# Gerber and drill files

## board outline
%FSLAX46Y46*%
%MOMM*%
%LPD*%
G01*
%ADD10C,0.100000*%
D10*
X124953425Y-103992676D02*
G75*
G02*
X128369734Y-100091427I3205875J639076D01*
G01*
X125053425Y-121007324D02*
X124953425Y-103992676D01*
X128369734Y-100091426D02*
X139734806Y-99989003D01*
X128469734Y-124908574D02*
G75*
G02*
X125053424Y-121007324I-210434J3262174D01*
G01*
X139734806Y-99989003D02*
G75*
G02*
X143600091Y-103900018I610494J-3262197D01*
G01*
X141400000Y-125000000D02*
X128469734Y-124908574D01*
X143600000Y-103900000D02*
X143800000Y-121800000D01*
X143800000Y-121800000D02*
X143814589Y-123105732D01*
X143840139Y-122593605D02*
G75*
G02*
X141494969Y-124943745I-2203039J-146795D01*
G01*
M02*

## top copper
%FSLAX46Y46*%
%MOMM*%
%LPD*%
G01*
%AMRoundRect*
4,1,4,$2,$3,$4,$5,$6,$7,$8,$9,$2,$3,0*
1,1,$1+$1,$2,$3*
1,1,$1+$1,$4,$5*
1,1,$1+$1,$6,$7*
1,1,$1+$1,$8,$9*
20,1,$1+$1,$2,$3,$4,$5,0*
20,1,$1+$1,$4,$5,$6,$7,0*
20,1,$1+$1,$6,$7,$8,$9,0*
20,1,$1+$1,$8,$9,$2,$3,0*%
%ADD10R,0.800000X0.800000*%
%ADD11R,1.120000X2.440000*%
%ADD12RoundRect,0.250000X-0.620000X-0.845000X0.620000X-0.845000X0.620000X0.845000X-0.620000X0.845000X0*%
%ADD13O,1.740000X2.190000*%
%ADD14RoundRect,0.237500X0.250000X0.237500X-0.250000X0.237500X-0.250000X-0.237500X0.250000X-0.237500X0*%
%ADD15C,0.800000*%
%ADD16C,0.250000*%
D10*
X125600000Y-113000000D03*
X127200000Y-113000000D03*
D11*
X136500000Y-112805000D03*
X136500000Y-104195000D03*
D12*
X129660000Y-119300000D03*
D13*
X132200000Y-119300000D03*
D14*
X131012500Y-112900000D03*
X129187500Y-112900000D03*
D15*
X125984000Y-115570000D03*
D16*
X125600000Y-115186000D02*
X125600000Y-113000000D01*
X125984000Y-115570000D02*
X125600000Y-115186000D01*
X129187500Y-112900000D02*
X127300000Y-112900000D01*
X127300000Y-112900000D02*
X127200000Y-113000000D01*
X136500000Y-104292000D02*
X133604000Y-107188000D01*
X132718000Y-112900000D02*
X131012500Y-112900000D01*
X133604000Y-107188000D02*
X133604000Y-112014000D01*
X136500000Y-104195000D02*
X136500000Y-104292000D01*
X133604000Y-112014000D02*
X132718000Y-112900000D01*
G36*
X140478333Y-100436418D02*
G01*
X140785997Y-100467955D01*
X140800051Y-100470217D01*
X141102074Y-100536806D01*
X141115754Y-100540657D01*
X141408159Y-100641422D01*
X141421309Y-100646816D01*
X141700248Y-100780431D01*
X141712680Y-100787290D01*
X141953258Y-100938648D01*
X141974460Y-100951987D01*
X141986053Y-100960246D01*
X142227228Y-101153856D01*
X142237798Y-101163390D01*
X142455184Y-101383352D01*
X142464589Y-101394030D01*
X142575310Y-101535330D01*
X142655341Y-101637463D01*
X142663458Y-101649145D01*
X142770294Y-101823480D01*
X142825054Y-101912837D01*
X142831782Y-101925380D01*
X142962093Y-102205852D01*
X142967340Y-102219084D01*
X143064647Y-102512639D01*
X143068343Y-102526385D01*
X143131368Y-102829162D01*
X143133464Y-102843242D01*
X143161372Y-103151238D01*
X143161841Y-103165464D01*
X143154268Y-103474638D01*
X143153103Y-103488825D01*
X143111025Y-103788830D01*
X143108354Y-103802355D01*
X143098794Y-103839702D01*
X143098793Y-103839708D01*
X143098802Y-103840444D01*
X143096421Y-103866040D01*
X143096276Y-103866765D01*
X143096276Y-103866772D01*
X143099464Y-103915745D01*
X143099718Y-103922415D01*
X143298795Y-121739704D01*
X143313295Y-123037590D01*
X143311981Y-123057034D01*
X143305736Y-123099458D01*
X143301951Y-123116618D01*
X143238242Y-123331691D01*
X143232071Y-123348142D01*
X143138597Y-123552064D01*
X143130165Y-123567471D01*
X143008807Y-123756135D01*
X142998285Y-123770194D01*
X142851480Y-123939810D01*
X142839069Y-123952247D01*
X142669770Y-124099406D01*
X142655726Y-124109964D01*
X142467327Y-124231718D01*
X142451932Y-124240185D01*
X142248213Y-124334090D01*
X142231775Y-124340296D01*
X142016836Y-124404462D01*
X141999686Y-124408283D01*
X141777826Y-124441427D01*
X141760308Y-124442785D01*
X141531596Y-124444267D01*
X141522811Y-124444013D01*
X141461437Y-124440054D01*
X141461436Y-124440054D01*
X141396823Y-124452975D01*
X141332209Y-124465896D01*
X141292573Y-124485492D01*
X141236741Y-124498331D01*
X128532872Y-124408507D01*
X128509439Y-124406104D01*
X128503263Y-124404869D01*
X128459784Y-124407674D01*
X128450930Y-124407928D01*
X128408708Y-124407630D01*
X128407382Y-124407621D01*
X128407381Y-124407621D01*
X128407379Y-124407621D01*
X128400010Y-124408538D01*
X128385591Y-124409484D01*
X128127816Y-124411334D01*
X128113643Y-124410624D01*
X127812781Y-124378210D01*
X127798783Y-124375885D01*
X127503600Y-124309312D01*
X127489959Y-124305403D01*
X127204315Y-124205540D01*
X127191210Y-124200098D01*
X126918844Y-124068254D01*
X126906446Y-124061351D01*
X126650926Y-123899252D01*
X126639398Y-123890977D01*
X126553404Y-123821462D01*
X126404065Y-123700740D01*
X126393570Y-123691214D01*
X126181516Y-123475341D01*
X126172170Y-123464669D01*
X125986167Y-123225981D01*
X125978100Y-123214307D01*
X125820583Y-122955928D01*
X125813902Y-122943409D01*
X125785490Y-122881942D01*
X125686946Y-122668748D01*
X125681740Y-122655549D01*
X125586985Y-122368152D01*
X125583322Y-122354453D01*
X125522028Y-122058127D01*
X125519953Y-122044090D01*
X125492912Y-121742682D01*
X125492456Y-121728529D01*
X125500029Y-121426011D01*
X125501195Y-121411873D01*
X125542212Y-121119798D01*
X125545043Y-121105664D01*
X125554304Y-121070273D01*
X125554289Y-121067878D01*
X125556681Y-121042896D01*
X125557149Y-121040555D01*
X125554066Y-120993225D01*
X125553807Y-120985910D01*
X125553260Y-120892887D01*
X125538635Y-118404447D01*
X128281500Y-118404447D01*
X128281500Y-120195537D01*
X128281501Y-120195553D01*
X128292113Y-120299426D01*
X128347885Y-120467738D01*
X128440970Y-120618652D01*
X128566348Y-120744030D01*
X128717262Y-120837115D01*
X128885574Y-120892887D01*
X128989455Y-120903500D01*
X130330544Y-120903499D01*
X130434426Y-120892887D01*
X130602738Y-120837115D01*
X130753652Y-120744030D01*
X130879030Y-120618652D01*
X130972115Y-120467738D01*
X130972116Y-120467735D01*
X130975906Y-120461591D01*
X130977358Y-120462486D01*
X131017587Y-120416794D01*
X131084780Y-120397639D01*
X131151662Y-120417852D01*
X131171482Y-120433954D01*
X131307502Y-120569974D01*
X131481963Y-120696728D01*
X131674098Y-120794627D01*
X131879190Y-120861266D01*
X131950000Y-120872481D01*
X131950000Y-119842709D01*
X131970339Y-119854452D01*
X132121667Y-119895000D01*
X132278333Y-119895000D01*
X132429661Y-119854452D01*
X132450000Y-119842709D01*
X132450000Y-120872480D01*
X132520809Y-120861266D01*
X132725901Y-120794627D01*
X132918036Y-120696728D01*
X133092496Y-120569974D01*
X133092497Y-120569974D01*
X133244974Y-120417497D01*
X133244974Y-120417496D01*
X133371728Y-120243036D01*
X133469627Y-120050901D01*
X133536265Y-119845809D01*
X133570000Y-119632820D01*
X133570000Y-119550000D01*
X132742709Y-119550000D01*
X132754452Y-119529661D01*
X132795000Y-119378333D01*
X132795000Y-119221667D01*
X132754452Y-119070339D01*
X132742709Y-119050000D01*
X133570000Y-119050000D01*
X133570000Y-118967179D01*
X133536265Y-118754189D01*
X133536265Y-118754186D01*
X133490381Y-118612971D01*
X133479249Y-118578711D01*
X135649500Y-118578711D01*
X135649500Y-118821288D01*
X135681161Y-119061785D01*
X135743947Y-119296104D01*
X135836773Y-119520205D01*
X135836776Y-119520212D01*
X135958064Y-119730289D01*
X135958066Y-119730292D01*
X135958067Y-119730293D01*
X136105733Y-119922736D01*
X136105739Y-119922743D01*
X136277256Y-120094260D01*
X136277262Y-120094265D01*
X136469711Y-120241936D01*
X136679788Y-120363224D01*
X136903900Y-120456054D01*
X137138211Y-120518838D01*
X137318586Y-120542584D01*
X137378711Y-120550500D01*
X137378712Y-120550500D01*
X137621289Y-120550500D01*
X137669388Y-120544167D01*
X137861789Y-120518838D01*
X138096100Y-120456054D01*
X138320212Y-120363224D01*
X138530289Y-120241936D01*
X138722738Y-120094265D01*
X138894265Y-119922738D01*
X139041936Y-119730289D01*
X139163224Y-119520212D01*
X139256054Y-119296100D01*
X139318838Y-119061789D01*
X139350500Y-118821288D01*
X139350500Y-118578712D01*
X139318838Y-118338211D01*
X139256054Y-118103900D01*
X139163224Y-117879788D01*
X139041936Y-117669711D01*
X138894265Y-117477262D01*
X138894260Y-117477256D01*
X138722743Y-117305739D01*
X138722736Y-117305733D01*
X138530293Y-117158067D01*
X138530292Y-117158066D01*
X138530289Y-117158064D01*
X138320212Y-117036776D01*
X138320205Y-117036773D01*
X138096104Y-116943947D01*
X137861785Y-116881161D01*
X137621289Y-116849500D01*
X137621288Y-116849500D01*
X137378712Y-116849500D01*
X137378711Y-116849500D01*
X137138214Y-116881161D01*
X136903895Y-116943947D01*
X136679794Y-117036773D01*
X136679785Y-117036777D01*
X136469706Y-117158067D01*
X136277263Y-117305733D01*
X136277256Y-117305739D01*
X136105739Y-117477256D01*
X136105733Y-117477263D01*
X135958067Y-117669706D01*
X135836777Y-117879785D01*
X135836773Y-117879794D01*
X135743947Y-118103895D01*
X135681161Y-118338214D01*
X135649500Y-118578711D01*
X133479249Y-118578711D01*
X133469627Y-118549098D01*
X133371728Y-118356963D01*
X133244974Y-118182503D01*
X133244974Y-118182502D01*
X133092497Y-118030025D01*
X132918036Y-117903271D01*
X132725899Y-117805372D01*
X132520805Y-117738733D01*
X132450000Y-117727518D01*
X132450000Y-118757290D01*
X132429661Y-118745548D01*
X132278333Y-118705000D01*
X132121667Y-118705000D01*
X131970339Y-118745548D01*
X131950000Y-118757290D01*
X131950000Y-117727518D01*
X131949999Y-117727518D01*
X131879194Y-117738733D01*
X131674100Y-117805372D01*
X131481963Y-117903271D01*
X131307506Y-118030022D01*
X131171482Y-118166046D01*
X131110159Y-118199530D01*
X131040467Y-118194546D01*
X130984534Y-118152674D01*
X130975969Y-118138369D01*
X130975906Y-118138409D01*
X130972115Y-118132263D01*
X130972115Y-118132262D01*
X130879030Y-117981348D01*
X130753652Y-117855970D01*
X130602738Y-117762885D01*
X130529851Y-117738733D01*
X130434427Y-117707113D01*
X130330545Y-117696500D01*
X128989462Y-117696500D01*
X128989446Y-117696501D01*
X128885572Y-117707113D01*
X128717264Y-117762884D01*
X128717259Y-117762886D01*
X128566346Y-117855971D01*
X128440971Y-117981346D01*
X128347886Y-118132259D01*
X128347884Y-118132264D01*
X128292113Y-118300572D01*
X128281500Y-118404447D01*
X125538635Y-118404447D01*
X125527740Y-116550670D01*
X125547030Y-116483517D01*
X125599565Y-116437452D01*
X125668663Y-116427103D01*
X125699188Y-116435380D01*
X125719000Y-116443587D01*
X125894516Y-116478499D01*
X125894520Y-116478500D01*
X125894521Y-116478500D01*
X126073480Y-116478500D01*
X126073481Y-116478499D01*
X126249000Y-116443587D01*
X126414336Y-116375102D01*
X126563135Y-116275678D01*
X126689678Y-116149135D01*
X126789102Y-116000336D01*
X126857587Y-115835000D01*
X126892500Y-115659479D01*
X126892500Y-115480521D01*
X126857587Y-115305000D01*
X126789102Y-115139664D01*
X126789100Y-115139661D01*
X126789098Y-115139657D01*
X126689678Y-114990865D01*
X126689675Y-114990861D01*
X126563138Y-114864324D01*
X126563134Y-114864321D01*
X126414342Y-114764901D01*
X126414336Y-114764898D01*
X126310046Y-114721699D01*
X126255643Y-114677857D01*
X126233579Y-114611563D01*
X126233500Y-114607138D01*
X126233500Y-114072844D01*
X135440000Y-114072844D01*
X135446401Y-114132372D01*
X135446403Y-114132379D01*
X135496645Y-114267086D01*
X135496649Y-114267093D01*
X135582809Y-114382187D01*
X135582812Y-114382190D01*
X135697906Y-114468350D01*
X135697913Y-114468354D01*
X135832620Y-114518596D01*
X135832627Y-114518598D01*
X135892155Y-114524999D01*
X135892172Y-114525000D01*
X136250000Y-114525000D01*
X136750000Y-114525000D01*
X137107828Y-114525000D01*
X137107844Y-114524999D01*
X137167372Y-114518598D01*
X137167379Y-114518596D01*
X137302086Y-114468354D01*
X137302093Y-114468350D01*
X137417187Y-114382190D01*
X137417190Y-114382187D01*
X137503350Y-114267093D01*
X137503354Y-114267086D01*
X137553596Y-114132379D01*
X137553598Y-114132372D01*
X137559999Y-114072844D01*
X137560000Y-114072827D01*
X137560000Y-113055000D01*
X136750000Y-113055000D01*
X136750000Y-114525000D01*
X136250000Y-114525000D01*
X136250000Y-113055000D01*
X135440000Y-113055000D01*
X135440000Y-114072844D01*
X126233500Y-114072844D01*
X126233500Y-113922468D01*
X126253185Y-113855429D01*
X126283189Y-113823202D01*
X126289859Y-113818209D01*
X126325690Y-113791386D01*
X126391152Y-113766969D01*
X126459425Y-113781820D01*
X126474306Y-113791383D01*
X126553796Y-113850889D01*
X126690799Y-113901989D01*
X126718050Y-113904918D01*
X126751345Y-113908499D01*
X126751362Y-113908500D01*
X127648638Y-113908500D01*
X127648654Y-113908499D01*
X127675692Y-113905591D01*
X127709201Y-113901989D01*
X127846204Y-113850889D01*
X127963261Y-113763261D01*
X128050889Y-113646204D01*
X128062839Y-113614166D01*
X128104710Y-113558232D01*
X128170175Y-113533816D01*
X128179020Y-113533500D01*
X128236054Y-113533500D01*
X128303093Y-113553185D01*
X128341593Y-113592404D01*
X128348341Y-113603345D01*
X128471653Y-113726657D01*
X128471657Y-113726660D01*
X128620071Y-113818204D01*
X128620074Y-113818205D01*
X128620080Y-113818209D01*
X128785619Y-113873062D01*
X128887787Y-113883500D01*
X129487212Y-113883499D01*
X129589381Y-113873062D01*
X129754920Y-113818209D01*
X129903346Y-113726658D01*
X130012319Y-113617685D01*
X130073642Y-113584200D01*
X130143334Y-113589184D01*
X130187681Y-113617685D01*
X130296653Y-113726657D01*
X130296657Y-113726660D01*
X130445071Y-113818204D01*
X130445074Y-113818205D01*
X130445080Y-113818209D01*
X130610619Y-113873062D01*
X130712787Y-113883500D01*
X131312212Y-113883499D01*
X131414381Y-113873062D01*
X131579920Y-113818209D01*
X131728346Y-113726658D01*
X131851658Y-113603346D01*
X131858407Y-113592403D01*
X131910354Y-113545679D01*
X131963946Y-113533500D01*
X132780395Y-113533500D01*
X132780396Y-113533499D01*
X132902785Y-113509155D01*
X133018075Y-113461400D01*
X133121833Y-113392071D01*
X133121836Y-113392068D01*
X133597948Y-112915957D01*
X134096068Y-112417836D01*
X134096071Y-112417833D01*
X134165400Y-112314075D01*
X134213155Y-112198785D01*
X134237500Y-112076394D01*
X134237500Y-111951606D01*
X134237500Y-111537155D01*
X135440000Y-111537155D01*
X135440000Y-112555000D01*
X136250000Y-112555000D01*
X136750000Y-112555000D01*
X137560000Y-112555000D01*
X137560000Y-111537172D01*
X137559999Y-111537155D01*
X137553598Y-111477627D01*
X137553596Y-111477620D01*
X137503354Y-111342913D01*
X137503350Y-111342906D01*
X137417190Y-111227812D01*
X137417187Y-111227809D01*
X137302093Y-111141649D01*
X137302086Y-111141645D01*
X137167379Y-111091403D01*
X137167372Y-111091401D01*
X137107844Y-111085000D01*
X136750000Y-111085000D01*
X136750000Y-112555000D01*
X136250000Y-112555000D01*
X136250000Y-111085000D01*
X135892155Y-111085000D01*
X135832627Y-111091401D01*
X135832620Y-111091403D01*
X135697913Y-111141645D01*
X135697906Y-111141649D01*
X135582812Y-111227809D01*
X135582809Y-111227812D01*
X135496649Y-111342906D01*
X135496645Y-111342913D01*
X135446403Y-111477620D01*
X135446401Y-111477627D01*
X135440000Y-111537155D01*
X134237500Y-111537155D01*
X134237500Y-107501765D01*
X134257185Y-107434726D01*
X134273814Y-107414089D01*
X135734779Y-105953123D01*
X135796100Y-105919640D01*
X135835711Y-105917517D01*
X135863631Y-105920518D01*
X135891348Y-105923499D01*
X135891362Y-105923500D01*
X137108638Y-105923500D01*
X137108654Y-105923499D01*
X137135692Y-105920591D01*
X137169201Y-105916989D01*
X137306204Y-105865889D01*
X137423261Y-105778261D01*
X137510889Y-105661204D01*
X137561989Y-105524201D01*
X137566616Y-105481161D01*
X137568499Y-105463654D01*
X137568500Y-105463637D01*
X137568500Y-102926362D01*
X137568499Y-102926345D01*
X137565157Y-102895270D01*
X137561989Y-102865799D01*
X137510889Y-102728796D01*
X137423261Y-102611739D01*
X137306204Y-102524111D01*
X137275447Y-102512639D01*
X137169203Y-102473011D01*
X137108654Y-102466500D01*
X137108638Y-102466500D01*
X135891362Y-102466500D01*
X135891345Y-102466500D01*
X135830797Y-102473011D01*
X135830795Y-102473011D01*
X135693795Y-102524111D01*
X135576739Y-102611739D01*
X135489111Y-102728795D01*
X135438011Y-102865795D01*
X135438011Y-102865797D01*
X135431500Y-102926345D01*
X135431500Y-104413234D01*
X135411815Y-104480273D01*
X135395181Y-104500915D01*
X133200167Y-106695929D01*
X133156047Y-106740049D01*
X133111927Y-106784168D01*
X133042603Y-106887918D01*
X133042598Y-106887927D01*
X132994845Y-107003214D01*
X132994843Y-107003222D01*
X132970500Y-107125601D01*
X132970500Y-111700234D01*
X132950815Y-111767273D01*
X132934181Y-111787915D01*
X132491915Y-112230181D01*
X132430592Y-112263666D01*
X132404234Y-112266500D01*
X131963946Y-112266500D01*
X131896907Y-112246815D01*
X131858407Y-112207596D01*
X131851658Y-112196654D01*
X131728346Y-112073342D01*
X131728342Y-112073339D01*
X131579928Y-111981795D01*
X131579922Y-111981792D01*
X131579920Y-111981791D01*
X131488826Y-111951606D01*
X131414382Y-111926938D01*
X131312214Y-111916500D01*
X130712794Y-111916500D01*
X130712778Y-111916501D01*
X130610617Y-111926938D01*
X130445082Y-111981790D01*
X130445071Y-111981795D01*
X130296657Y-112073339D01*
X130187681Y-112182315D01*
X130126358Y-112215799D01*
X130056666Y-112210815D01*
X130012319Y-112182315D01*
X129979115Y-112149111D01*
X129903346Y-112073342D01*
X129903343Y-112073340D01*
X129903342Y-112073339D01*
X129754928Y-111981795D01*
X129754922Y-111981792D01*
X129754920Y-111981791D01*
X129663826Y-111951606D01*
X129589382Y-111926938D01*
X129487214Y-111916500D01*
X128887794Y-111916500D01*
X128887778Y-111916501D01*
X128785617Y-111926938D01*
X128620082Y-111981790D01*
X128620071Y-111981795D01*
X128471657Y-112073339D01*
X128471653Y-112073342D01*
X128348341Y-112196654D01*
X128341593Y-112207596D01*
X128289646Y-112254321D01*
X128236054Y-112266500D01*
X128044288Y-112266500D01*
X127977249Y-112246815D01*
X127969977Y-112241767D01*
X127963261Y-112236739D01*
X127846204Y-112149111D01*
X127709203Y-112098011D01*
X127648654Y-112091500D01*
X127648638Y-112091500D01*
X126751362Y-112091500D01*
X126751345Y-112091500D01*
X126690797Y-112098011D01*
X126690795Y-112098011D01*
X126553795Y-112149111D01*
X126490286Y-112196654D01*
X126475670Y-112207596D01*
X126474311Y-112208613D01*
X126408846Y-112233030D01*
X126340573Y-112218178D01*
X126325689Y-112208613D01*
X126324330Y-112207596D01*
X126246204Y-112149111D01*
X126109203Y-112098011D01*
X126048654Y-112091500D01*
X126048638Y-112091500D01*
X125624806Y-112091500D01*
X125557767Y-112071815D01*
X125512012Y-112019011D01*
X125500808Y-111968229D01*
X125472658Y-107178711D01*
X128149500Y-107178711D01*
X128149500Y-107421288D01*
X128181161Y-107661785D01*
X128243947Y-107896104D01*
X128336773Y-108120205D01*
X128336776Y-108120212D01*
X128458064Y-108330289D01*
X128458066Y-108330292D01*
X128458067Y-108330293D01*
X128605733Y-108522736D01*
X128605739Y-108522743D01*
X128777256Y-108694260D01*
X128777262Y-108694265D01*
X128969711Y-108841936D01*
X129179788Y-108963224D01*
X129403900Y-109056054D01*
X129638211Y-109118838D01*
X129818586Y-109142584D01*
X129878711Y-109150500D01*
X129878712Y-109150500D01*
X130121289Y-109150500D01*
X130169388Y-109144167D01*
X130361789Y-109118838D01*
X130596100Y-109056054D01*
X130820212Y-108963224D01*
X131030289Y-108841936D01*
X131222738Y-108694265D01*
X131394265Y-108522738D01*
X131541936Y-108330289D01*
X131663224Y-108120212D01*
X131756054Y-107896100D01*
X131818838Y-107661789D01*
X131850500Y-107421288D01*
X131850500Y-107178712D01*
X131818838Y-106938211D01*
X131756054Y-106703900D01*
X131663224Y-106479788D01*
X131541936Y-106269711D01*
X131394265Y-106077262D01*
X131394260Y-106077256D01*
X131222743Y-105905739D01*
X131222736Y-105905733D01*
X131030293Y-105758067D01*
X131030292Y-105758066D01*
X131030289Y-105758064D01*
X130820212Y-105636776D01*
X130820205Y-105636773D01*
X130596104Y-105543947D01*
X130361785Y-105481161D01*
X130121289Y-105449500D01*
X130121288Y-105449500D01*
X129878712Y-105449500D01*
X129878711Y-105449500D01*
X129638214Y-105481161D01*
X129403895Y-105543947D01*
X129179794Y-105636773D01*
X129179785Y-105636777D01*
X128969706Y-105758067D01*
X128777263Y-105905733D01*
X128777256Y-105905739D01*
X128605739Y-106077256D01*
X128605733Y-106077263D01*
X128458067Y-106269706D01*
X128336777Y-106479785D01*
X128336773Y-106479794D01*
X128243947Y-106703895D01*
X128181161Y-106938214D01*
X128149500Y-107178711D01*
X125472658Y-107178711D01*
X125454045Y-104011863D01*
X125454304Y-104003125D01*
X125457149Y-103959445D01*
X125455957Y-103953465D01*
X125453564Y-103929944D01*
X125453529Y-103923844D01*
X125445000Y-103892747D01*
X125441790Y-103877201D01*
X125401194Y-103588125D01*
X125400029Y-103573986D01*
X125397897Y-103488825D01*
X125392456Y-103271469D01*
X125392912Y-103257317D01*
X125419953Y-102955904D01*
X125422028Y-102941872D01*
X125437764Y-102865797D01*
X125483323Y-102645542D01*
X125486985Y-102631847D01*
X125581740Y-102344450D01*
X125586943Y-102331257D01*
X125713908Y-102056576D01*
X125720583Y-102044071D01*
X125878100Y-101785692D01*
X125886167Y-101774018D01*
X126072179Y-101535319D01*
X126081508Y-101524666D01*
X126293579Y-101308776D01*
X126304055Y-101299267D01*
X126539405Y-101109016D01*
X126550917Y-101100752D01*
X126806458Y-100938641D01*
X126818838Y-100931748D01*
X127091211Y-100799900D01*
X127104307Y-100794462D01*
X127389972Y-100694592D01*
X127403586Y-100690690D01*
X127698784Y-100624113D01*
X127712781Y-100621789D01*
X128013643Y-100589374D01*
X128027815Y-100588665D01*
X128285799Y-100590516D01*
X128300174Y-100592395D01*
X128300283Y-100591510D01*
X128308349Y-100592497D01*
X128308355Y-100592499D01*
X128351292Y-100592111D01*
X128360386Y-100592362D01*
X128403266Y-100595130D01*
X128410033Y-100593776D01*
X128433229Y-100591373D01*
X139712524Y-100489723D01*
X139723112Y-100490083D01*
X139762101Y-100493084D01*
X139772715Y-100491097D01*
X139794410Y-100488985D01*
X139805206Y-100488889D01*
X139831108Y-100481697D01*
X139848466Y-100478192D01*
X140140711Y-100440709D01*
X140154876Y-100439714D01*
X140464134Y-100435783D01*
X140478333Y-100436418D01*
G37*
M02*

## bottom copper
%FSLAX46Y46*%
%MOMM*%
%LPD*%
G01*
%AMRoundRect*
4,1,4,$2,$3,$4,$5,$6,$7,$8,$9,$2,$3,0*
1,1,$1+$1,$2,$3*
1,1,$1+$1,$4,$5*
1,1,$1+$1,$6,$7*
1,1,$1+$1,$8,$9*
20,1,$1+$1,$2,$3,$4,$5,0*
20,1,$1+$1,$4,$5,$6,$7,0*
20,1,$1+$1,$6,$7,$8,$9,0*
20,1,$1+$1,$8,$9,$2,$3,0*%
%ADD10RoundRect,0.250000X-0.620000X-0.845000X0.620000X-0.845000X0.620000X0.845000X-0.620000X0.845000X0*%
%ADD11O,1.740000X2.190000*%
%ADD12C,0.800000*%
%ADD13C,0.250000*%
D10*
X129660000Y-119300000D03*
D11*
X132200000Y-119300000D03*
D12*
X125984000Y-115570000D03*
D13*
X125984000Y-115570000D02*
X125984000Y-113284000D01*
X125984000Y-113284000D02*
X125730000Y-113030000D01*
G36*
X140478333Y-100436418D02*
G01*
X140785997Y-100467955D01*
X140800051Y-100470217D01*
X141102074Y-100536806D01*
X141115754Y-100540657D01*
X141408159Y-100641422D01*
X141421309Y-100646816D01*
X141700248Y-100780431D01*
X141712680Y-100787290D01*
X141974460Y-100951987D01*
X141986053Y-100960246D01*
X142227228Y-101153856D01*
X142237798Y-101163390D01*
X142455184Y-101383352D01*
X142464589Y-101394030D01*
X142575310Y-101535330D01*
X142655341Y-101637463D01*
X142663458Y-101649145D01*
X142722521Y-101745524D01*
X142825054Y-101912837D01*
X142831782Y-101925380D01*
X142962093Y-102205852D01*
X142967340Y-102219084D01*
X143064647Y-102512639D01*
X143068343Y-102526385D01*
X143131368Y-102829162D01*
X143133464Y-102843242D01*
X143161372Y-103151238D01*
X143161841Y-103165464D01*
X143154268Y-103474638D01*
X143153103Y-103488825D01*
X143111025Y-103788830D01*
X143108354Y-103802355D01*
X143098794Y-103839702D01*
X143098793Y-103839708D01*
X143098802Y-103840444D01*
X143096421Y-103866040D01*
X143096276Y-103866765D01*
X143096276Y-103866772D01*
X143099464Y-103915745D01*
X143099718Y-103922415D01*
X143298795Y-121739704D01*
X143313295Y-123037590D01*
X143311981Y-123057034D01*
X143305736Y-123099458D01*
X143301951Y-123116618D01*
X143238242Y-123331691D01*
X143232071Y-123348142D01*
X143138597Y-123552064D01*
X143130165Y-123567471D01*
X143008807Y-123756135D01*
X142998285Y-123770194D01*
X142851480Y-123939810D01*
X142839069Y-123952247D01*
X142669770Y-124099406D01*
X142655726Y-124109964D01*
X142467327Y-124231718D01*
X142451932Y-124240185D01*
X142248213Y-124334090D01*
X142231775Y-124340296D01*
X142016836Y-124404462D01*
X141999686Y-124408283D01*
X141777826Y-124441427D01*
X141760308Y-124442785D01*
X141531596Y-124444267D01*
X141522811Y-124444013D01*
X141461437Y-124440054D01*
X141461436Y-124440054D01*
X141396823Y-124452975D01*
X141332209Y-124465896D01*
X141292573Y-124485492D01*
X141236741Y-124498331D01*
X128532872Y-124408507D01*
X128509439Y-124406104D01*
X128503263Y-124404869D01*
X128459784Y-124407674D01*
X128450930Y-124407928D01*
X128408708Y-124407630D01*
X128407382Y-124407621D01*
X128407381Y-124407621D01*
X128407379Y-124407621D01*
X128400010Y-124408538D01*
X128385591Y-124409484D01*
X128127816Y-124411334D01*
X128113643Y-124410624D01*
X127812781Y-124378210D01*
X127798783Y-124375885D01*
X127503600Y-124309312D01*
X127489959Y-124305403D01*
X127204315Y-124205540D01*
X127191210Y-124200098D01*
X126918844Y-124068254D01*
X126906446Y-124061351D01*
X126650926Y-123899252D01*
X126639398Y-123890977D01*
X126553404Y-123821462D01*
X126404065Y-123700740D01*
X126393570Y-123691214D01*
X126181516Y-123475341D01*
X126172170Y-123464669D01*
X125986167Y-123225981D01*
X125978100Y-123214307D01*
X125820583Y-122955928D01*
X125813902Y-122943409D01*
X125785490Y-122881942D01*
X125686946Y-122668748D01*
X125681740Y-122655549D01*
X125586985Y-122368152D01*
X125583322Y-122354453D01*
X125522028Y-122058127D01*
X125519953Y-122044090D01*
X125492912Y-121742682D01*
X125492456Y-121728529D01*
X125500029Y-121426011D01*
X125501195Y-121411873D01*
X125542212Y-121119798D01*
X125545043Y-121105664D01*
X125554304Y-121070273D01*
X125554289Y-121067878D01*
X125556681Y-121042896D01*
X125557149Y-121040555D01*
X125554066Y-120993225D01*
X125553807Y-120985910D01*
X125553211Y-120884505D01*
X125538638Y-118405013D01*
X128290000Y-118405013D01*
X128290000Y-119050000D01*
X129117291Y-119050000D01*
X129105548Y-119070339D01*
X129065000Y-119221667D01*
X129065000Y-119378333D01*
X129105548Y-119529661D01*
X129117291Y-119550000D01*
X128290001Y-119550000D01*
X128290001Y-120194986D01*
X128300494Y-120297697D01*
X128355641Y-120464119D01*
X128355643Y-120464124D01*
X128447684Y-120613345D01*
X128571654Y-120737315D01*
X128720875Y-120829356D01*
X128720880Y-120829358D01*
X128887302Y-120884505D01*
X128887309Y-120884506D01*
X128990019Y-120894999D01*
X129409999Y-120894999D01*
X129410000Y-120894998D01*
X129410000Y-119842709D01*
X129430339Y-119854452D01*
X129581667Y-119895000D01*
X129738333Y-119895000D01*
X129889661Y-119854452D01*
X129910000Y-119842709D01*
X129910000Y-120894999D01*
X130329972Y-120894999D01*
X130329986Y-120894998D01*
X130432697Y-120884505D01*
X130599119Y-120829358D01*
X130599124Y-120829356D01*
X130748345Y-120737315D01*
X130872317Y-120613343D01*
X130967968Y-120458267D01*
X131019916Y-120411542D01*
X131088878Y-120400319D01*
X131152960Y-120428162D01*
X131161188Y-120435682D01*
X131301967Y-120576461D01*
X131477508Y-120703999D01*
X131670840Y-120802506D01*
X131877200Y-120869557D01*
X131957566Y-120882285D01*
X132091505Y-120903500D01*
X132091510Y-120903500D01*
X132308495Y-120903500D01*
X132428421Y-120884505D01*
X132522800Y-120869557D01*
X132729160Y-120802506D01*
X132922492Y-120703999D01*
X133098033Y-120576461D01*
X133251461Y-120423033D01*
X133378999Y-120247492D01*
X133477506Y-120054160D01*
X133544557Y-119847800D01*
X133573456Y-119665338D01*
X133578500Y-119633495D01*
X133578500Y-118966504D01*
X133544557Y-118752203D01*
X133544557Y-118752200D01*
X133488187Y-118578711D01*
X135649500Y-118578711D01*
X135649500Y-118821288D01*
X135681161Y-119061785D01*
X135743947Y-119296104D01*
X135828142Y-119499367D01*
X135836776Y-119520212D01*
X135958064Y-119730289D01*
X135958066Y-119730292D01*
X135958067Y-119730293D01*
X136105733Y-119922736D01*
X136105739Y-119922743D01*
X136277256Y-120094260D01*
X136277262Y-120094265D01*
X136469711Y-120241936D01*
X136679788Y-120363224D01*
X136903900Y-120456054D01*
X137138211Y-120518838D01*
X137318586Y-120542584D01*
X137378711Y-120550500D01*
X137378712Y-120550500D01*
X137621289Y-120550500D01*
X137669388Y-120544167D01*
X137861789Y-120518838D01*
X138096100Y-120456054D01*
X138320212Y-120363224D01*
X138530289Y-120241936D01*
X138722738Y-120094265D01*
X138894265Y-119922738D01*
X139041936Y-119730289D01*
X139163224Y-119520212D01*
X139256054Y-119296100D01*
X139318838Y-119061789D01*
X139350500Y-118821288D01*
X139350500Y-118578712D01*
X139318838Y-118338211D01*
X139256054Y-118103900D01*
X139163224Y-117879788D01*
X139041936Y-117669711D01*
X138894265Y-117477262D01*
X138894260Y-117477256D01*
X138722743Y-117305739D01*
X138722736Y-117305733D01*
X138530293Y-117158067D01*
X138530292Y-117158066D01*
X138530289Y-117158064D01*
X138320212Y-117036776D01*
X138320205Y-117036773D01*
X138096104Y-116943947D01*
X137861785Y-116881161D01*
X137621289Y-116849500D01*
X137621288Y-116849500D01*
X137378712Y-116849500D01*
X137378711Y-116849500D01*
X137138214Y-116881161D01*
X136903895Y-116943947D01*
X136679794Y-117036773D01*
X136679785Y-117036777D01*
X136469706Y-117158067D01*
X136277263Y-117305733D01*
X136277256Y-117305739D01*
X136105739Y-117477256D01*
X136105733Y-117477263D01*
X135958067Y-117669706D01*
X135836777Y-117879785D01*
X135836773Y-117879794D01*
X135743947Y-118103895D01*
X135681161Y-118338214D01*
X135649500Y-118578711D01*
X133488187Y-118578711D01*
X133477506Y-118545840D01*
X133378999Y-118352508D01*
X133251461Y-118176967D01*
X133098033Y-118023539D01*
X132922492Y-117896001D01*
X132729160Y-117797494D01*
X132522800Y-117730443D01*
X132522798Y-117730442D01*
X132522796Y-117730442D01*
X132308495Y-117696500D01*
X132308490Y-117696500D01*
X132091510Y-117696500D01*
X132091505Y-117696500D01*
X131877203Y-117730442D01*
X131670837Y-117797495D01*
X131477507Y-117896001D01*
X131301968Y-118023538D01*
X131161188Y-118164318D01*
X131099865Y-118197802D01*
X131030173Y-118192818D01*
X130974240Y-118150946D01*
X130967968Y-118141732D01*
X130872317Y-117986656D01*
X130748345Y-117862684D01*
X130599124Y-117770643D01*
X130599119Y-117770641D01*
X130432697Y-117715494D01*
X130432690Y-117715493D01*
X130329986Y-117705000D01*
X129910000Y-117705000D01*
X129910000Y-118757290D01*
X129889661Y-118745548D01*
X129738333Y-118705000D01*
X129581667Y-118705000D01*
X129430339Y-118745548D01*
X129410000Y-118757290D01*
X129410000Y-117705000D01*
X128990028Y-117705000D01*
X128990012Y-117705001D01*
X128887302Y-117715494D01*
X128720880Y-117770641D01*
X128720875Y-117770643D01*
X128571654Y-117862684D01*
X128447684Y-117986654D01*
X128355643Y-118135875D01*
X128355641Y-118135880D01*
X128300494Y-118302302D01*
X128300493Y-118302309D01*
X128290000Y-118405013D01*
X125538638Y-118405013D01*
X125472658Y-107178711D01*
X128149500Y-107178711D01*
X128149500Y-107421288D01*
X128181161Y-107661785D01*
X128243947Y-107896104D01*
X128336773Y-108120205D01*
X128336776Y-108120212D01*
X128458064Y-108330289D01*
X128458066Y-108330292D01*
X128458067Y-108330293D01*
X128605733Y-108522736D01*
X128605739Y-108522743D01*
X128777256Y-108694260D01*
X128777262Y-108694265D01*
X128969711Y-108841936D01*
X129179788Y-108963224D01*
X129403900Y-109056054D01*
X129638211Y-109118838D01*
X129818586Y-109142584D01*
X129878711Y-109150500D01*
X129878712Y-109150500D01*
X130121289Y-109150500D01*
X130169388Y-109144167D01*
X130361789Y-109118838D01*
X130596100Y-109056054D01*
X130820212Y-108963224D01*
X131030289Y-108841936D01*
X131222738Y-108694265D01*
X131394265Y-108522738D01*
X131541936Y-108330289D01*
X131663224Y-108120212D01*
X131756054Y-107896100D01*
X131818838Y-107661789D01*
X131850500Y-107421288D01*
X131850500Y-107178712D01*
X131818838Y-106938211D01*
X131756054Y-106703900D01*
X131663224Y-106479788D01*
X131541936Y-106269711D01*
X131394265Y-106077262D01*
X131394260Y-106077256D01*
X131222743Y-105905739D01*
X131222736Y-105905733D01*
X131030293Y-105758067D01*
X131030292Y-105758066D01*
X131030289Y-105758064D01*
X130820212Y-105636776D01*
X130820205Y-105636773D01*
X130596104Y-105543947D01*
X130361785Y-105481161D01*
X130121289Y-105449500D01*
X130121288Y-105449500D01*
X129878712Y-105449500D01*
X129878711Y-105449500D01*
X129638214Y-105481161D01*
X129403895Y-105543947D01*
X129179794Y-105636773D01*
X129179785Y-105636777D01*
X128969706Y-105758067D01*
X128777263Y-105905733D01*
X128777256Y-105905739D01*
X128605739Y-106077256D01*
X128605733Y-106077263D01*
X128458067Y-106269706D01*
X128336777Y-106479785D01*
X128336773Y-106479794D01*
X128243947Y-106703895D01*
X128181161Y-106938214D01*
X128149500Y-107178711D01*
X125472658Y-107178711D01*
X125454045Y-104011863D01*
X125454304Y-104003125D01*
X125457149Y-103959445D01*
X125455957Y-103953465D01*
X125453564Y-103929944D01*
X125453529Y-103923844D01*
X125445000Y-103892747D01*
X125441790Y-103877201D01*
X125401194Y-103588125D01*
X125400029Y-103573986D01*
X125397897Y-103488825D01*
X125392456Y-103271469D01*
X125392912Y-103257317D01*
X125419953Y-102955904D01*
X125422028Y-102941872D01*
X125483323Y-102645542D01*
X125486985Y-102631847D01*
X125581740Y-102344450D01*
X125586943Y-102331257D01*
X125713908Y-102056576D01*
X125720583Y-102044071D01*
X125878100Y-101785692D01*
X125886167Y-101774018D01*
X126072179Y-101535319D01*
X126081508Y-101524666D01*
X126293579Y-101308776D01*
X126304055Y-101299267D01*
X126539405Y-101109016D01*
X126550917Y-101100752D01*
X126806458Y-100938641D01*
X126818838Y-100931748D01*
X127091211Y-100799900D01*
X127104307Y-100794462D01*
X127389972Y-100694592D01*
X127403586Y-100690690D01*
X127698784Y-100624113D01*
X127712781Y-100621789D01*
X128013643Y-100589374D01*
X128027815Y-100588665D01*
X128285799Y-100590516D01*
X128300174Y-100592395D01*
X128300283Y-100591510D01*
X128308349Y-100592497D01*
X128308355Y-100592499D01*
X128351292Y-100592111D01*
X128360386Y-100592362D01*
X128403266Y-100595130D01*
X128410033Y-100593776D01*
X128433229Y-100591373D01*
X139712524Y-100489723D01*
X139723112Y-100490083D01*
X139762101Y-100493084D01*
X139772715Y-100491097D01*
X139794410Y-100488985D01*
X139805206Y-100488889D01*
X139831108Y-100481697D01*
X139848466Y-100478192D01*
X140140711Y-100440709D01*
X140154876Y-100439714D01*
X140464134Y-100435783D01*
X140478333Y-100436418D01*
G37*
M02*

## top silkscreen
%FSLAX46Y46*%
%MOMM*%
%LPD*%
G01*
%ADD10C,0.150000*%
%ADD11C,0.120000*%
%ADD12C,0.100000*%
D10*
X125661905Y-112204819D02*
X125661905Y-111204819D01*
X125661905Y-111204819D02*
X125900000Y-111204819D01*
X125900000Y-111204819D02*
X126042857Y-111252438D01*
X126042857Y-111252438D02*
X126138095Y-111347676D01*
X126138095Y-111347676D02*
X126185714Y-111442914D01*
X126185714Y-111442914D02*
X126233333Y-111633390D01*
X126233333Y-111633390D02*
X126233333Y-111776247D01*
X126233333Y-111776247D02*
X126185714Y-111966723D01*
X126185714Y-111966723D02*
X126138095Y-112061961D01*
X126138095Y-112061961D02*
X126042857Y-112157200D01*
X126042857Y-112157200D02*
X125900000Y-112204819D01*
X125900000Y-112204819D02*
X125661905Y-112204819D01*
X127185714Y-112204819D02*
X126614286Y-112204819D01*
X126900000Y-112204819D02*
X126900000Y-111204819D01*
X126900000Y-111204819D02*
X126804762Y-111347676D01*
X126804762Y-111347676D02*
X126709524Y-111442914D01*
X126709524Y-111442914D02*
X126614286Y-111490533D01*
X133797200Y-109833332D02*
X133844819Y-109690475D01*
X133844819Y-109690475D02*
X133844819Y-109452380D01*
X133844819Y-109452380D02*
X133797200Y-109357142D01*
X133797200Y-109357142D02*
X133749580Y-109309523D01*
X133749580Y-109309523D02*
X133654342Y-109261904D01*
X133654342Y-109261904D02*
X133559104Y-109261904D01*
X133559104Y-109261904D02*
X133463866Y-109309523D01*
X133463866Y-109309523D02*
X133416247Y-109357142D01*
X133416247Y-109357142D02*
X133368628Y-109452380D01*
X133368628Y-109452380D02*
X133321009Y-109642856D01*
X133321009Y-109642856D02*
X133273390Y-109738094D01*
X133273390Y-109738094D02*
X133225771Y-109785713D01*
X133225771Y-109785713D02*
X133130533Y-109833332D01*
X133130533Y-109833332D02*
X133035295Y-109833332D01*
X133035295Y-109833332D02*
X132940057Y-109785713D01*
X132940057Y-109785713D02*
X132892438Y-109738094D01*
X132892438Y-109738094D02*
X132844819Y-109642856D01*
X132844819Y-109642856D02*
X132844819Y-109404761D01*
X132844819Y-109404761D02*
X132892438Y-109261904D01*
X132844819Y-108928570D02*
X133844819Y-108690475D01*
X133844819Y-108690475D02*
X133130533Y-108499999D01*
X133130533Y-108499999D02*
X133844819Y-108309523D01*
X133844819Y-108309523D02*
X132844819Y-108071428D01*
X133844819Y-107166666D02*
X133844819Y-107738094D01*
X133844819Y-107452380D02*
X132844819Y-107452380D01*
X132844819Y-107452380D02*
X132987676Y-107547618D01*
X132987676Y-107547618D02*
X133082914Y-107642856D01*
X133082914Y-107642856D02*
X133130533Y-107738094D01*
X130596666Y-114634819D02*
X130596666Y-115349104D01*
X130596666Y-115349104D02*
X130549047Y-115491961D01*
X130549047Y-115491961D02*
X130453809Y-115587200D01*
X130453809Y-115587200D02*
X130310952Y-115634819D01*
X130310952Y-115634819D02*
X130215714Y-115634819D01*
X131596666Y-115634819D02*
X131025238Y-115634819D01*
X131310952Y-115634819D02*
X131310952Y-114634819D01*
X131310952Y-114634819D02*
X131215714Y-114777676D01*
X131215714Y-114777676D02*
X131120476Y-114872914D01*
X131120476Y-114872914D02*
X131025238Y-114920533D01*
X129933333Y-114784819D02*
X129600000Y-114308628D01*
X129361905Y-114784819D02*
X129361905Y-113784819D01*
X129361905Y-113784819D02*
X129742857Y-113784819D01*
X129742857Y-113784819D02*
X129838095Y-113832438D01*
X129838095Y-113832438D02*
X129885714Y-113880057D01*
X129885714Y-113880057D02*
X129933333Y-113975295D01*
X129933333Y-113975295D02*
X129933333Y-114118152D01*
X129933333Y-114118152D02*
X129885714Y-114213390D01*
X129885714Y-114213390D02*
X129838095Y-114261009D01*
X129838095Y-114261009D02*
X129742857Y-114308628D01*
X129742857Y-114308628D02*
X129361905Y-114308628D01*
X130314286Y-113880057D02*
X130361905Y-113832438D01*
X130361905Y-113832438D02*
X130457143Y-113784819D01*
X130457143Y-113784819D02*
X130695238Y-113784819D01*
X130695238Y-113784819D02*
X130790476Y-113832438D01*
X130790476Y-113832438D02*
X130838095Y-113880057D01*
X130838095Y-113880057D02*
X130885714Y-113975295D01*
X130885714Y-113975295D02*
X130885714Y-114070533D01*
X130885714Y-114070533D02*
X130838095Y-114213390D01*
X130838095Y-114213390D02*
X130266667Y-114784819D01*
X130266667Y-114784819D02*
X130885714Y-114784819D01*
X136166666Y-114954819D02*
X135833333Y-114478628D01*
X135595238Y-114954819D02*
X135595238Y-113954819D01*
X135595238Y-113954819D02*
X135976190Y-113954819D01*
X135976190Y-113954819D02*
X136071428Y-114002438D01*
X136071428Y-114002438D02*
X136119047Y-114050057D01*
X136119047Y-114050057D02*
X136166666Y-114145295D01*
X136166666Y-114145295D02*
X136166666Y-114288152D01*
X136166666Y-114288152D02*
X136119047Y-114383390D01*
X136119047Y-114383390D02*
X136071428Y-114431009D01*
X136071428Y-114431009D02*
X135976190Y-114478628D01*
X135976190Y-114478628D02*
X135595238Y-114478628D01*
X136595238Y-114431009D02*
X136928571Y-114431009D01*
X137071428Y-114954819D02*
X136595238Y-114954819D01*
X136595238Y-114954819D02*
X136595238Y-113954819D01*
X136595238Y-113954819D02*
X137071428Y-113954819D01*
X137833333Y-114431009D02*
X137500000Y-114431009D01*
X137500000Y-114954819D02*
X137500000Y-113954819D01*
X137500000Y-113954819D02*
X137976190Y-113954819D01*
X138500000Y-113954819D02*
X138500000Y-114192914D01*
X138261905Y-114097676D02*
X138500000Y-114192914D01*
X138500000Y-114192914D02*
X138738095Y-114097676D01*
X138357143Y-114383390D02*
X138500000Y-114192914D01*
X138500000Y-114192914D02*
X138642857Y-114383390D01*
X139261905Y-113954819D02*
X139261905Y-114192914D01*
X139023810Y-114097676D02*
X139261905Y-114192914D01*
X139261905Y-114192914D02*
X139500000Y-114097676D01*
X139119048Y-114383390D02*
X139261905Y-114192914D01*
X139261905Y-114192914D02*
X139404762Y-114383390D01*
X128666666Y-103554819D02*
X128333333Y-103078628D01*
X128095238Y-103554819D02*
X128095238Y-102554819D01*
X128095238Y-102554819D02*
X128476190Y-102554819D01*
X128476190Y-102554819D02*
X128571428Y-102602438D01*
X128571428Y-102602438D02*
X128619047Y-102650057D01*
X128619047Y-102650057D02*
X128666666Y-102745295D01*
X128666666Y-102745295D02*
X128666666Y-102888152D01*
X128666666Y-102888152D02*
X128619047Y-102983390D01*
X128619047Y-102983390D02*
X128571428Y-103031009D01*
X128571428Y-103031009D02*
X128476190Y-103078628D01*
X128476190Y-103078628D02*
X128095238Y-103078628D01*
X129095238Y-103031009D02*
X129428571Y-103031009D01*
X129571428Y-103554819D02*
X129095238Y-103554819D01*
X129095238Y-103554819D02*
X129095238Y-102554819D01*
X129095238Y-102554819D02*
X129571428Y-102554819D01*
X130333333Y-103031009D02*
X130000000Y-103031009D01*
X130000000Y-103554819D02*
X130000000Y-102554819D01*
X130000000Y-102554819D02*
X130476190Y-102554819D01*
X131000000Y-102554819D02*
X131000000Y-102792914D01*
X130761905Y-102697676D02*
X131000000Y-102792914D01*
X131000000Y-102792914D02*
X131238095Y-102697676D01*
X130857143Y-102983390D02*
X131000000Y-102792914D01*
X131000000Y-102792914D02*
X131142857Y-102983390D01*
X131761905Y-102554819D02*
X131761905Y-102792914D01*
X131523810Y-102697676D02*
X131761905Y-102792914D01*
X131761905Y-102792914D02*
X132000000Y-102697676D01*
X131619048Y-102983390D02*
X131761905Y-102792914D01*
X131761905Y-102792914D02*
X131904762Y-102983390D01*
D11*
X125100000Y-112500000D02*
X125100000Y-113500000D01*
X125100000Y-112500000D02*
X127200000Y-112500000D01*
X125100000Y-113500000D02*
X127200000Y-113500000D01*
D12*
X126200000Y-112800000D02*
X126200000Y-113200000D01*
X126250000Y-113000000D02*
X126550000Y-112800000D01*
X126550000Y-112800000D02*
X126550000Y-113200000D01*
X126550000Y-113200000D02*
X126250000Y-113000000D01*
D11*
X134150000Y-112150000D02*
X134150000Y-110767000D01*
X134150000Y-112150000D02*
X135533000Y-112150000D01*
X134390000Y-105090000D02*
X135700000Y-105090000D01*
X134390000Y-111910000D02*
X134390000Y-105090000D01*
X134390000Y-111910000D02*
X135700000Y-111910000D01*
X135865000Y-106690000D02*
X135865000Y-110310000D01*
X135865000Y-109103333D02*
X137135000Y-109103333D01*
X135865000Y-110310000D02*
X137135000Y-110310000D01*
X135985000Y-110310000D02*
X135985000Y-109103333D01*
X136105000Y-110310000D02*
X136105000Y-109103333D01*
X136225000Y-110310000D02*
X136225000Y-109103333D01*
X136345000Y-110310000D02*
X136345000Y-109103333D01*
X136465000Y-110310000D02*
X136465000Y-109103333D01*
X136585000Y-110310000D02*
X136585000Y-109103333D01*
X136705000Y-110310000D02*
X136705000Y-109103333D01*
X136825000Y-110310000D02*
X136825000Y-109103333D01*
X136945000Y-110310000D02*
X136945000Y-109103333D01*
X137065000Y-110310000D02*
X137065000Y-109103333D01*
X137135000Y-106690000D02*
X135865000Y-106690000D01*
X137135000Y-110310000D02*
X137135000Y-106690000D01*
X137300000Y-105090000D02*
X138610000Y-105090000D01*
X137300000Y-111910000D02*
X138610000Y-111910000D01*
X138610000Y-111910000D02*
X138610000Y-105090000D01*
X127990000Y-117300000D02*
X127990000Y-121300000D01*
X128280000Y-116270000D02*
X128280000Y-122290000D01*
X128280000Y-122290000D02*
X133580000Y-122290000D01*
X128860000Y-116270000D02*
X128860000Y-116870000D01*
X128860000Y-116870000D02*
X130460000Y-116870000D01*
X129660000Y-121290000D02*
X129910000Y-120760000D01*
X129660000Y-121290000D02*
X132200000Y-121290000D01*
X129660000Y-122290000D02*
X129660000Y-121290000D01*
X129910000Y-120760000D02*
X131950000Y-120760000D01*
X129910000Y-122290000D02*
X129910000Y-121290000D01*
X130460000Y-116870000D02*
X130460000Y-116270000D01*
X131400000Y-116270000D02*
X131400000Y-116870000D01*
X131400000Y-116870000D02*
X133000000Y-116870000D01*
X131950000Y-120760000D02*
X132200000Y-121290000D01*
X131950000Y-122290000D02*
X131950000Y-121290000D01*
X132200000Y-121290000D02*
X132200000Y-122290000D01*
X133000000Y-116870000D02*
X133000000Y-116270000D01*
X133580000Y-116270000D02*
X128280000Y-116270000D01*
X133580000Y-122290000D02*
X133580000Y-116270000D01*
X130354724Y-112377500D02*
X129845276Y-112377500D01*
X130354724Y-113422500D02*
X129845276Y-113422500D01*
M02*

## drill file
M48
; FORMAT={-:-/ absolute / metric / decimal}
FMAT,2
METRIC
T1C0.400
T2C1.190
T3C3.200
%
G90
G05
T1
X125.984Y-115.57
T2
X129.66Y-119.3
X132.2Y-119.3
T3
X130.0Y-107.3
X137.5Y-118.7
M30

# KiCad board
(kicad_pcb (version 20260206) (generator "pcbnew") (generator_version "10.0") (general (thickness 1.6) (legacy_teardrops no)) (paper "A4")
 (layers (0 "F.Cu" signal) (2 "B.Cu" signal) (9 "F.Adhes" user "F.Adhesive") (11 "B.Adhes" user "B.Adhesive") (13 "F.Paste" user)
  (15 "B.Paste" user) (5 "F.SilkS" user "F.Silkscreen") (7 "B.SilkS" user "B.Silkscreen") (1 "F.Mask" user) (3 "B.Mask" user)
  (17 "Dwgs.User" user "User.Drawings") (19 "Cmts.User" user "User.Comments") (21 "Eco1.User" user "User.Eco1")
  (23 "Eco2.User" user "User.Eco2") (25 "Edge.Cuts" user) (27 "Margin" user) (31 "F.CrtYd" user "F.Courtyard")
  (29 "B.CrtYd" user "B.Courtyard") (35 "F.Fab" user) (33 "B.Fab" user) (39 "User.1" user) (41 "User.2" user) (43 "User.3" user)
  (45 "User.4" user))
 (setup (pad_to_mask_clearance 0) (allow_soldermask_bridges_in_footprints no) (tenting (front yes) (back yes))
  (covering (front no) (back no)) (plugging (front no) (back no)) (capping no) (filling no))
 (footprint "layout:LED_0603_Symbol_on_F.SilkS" (layer "F.Cu") (at 126.4 113)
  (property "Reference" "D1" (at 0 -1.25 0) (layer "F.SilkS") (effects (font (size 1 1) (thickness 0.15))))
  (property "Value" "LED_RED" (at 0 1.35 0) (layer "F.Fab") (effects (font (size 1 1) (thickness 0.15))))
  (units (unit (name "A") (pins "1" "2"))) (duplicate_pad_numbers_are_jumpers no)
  (fp_line (start -1.3 -0.5) (end -1.3 0.5) (stroke (width 0.12) (type solid)) (layer "F.SilkS"))
  (fp_line (start -1.3 -0.5) (end 0.8 -0.5) (stroke (width 0.12) (type solid)) (layer "F.SilkS"))
  (fp_line (start -1.3 0.5) (end 0.8 0.5) (stroke (width 0.12) (type solid)) (layer "F.SilkS"))
  (fp_line (start -0.2 -0.2) (end -0.2 0.2) (stroke (width 0.1) (type solid)) (layer "F.SilkS"))
  (fp_line (start -0.15 0) (end 0.15 -0.2) (stroke (width 0.1) (type solid)) (layer "F.SilkS"))
  (fp_line (start 0.15 -0.2) (end 0.15 0.2) (stroke (width 0.1) (type solid)) (layer "F.SilkS"))
  (fp_line (start 0.15 0.2) (end -0.15 0) (stroke (width 0.1) (type solid)) (layer "F.SilkS"))
  (pad "1" smd rect (at -0.8 0 180) (size 0.8 0.8) (layers "F.Cu" "F.Mask" "F.Paste") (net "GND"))
  (pad "2" smd rect (at 0.8 0 180) (size 0.8 0.8) (layers "F.Cu" "F.Mask" "F.Paste") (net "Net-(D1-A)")))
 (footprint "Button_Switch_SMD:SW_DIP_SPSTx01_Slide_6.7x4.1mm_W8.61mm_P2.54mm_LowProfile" (layer "F.Cu") (at 136.5 108.5 90)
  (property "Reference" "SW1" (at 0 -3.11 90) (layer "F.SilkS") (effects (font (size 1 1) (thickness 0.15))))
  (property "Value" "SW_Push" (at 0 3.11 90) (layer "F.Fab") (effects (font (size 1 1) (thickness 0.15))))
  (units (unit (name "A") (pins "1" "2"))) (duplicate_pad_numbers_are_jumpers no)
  (fp_line (start -3.65 -2.35) (end -2.267 -2.35) (stroke (width 0.12) (type solid)) (layer "F.SilkS"))
  (fp_line (start -3.65 -2.35) (end -3.65 -0.967) (stroke (width 0.12) (type solid)) (layer "F.SilkS"))
  (fp_line (start 3.41 -2.11) (end 3.41 -0.8) (stroke (width 0.12) (type solid)) (layer "F.SilkS"))
  (fp_line (start -3.41 -2.11) (end 3.41 -2.11) (stroke (width 0.12) (type solid)) (layer "F.SilkS"))
  (fp_line (start -3.41 -2.11) (end -3.41 -0.8) (stroke (width 0.12) (type solid)) (layer "F.SilkS"))
  (fp_line (start 1.81 -0.635) (end -1.81 -0.635) (stroke (width 0.12) (type solid)) (layer "F.SilkS"))
  (fp_line (start -0.603333 -0.635) (end -0.603333 0.635) (stroke (width 0.12) (type solid)) (layer "F.SilkS"))
  (fp_line (start -1.81 -0.635) (end -1.81 0.635) (stroke (width 0.12) (type solid)) (layer "F.SilkS"))
  (fp_line (start -1.81 -0.515) (end -0.603333 -0.515) (stroke (width 0.12) (type solid)) (layer "F.SilkS"))
  (fp_line (start -1.81 -0.395) (end -0.603333 -0.395) (stroke (width 0.12) (type solid)) (layer "F.SilkS"))
  (fp_line (start -1.81 -0.275) (end -0.603333 -0.275) (stroke (width 0.12) (type solid)) (layer "F.SilkS"))
  (fp_line (start -1.81 -0.155) (end -0.603333 -0.155) (stroke (width 0.12) (type solid)) (layer "F.SilkS"))
  (fp_line (start -1.81 -0.035) (end -0.603333 -0.035) (stroke (width 0.12) (type solid)) (layer "F.SilkS"))
  (fp_line (start -1.81 0.085) (end -0.603333 0.085) (stroke (width 0.12) (type solid)) (layer "F.SilkS"))
  (fp_line (start -1.81 0.205) (end -0.603333 0.205) (stroke (width 0.12) (type solid)) (layer "F.SilkS"))
  (fp_line (start -1.81 0.325) (end -0.603333 0.325) (stroke (width 0.12) (type solid)) (layer "F.SilkS"))
  (fp_line (start -1.81 0.445) (end -0.603333 0.445) (stroke (width 0.12) (type solid)) (layer "F.SilkS"))
  (fp_line (start -1.81 0.565) (end -0.603333 0.565) (stroke (width 0.12) (type solid)) (layer "F.SilkS"))
  (fp_line (start 1.81 0.635) (end 1.81 -0.635) (stroke (width 0.12) (type solid)) (layer "F.SilkS"))
  (fp_line (start -1.81 0.635) (end 1.81 0.635) (stroke (width 0.12) (type solid)) (layer "F.SilkS"))
  (fp_line (start 3.41 0.8) (end 3.41 2.11) (stroke (width 0.12) (type solid)) (layer "F.SilkS"))
  (fp_line (start -3.41 0.8) (end -3.41 2.11) (stroke (width 0.12) (type solid)) (layer "F.SilkS"))
  (fp_line (start -3.41 2.11) (end 3.41 2.11) (stroke (width 0.12) (type solid)) (layer "F.SilkS"))
  (pad "1" smd rect (at -4.305 0 90) (size 2.44 1.12) (layers "F.Cu" "F.Mask" "F.Paste") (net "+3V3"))
  (pad "2" smd rect (at 4.305 0 90) (size 2.44 1.12) (layers "F.Cu" "F.Mask" "F.Paste") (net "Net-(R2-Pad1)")))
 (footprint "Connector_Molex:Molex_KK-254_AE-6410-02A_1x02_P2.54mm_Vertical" (layer "F.Cu") (at 129.66 119.3)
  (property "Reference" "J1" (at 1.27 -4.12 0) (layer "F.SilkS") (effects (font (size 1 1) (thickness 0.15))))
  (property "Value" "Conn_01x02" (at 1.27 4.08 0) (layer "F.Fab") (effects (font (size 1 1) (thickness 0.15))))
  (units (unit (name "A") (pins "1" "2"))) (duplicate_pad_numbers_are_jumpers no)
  (fp_line (start -1.67 -2) (end -1.67 2) (stroke (width 0.12) (type solid)) (layer "F.SilkS"))
  (fp_line (start -1.38 -3.03) (end -1.38 2.99) (stroke (width 0.12) (type solid)) (layer "F.SilkS"))
  (fp_line (start -1.38 2.99) (end 3.92 2.99) (stroke (width 0.12) (type solid)) (layer "F.SilkS"))
  (fp_line (start -0.8 -3.03) (end -0.8 -2.43) (stroke (width 0.12) (type solid)) (layer "F.SilkS"))
  (fp_line (start -0.8 -2.43) (end 0.8 -2.43) (stroke (width 0.12) (type solid)) (layer "F.SilkS"))
  (fp_line (start 0 1.99) (end 0.25 1.46) (stroke (width 0.12) (type solid)) (layer "F.SilkS"))
  (fp_line (start 0 1.99) (end 2.54 1.99) (stroke (width 0.12) (type solid)) (layer "F.SilkS"))
  (fp_line (start 0 2.99) (end 0 1.99) (stroke (width 0.12) (type solid)) (layer "F.SilkS"))
  (fp_line (start 0.25 1.46) (end 2.29 1.46) (stroke (width 0.12) (type solid)) (layer "F.SilkS"))
  (fp_line (start 0.25 2.99) (end 0.25 1.99) (stroke (width 0.12) (type solid)) (layer "F.SilkS"))
  (fp_line (start 0.8 -2.43) (end 0.8 -3.03) (stroke (width 0.12) (type solid)) (layer "F.SilkS"))
  (fp_line (start 1.74 -3.03) (end 1.74 -2.43) (stroke (width 0.12) (type solid)) (layer "F.SilkS"))
  (fp_line (start 1.74 -2.43) (end 3.34 -2.43) (stroke (width 0.12) (type solid)) (layer "F.SilkS"))
  (fp_line (start 2.29 1.46) (end 2.54 1.99) (stroke (width 0.12) (type solid)) (layer "F.SilkS"))
  (fp_line (start 2.29 2.99) (end 2.29 1.99) (stroke (width 0.12) (type solid)) (layer "F.SilkS"))
  (fp_line (start 2.54 1.99) (end 2.54 2.99) (stroke (width 0.12) (type solid)) (layer "F.SilkS"))
  (fp_line (start 3.34 -2.43) (end 3.34 -3.03) (stroke (width 0.12) (type solid)) (layer "F.SilkS"))
  (fp_line (start 3.92 -3.03) (end -1.38 -3.03) (stroke (width 0.12) (type solid)) (layer "F.SilkS"))
  (fp_line (start 3.92 2.99) (end 3.92 -3.03) (stroke (width 0.12) (type solid)) (layer "F.SilkS"))
  (pad "1" thru_hole roundrect (at 0 0) (size 1.74 2.19) (drill 1.19) (layers "*.Cu" "*.Mask") (remove_unused_layers no)
   (roundrect_rratio 0.143678) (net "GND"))
  (pad "2" thru_hole oval (at 2.54 0) (size 1.74 2.19) (drill 1.19) (layers "*.Cu" "*.Mask") (remove_unused_layers no) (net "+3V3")))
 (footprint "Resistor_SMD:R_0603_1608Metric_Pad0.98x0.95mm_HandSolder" (layer "F.Cu") (at 130.1 112.9 180)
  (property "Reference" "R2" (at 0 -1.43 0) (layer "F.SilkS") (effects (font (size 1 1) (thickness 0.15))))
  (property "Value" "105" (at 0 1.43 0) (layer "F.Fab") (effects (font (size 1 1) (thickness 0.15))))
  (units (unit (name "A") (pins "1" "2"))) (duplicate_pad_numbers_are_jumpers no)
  (fp_line (start -0.254724 0.5225) (end 0.254724 0.5225) (stroke (width 0.12) (type solid)) (layer "F.SilkS"))
  (fp_line (start -0.254724 -0.5225) (end 0.254724 -0.5225) (stroke (width 0.12) (type solid)) (layer "F.SilkS"))
  (pad "1" smd roundrect (at -0.9125 0 180) (size 0.975 0.95) (layers "F.Cu" "F.Mask" "F.Paste") (roundrect_rratio 0.25)
   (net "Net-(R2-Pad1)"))
  (pad "2" smd roundrect (at 0.9125 0 180) (size 0.975 0.95) (layers "F.Cu" "F.Mask" "F.Paste") (roundrect_rratio 0.25) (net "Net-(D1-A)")))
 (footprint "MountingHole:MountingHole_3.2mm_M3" (layer "F.Cu") (at 137.5 118.7)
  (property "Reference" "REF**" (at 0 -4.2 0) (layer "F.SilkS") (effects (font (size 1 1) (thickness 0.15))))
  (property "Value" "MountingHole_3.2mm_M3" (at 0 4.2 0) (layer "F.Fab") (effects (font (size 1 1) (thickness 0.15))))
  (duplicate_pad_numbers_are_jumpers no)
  (pad "" np_thru_hole circle (at 0 0) (size 3.2 3.2) (drill 3.2) (layers "*.Cu" "*.Mask")))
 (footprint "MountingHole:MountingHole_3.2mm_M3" (layer "F.Cu") (at 130 107.3)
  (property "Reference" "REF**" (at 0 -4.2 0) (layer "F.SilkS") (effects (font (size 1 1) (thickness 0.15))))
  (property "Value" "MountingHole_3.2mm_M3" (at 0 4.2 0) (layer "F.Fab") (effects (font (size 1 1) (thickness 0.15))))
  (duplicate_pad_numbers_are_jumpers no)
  (pad "" np_thru_hole circle (at 0 0) (size 3.2 3.2) (drill 3.2) (layers "*.Cu" "*.Mask")))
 (gr_arc (start 124.953425 103.992676) (mid 125.7 101.2) (end 128.369734 100.091426) (stroke (width 0.1) (type default)) (layer "Edge.Cuts"))
 (gr_line (start 125.053425 121.007324) (end 124.953425 103.992676) (stroke (width 0.1) (type default)) (layer "Edge.Cuts"))
 (gr_line (start 128.369734 100.091426) (end 139.734806 99.989003) (stroke (width 0.1) (type default)) (layer "Edge.Cuts"))
 (gr_arc (start 128.469734 124.908574) (mid 125.8 123.8) (end 125.053425 121.007324) (stroke (width 0.1) (type default)) (layer "Edge.Cuts"))
 (gr_arc (start 139.734806 99.989003) (mid 142.705779 100.918286) (end 143.6 103.9) (stroke (width 0.1) (type default)) (layer "Edge.Cuts"))
 (gr_line (start 141.4 125) (end 128.469734 124.908574) (stroke (width 0.1) (type default)) (layer "Edge.Cuts"))
 (gr_line (start 143.6 103.9) (end 143.8 121.8) (stroke (width 0.1) (type default)) (layer "Edge.Cuts"))
 (gr_line (start 143.8 121.8) (end 143.814589 123.105732) (stroke (width 0.1) (type default)) (layer "Edge.Cuts"))
 (gr_arc (start 143.840139 122.593605) (mid 143.2 124.3) (end 141.494968 124.943758) (stroke (width 0.1) (type default)) (layer "Edge.Cuts"))
 (segment (start 125.6 115.186) (end 125.6 113) (width 0.25) (layer "F.Cu") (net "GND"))
 (segment (start 125.984 115.57) (end 125.6 115.186) (width 0.25) (layer "F.Cu") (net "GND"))
 (via (at 125.984 115.57) (size 0.8) (drill 0.4) (layers "F.Cu" "B.Cu") (free yes) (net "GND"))
 (segment (start 125.984 115.57) (end 125.984 113.284) (width 0.25) (layer "B.Cu") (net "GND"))
 (segment (start 125.984 113.284) (end 125.73 113.03) (width 0.25) (layer "B.Cu") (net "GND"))
 (segment (start 129.1875 112.9) (end 127.3 112.9) (width 0.25) (layer "F.Cu") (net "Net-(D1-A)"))
 (segment (start 127.3 112.9) (end 127.2 113) (width 0.25) (layer "F.Cu") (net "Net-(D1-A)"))
 (segment (start 136.5 104.292) (end 133.604 107.188) (width 0.25) (layer "F.Cu") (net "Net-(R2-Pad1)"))
 (segment (start 132.718 112.9) (end 131.0125 112.9) (width 0.25) (layer "F.Cu") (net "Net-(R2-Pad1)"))
 (segment (start 133.604 107.188) (end 133.604 112.014) (width 0.25) (layer "F.Cu") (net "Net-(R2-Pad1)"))
 (segment (start 136.5 104.195) (end 136.5 104.292) (width 0.25) (layer "F.Cu") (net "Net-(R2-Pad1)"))
 (segment (start 133.604 112.014) (end 132.718 112.9) (width 0.25) (layer "F.Cu") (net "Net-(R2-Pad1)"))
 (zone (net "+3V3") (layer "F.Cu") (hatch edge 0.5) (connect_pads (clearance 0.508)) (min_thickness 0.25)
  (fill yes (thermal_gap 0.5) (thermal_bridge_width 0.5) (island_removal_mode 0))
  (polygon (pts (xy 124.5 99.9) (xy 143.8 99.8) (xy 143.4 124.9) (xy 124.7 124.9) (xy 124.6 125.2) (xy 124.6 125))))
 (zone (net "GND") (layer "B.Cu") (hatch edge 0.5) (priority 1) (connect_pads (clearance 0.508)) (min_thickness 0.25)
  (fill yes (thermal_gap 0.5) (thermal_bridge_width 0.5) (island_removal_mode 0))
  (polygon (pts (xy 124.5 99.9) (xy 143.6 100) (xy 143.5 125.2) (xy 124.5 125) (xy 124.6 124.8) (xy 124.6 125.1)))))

